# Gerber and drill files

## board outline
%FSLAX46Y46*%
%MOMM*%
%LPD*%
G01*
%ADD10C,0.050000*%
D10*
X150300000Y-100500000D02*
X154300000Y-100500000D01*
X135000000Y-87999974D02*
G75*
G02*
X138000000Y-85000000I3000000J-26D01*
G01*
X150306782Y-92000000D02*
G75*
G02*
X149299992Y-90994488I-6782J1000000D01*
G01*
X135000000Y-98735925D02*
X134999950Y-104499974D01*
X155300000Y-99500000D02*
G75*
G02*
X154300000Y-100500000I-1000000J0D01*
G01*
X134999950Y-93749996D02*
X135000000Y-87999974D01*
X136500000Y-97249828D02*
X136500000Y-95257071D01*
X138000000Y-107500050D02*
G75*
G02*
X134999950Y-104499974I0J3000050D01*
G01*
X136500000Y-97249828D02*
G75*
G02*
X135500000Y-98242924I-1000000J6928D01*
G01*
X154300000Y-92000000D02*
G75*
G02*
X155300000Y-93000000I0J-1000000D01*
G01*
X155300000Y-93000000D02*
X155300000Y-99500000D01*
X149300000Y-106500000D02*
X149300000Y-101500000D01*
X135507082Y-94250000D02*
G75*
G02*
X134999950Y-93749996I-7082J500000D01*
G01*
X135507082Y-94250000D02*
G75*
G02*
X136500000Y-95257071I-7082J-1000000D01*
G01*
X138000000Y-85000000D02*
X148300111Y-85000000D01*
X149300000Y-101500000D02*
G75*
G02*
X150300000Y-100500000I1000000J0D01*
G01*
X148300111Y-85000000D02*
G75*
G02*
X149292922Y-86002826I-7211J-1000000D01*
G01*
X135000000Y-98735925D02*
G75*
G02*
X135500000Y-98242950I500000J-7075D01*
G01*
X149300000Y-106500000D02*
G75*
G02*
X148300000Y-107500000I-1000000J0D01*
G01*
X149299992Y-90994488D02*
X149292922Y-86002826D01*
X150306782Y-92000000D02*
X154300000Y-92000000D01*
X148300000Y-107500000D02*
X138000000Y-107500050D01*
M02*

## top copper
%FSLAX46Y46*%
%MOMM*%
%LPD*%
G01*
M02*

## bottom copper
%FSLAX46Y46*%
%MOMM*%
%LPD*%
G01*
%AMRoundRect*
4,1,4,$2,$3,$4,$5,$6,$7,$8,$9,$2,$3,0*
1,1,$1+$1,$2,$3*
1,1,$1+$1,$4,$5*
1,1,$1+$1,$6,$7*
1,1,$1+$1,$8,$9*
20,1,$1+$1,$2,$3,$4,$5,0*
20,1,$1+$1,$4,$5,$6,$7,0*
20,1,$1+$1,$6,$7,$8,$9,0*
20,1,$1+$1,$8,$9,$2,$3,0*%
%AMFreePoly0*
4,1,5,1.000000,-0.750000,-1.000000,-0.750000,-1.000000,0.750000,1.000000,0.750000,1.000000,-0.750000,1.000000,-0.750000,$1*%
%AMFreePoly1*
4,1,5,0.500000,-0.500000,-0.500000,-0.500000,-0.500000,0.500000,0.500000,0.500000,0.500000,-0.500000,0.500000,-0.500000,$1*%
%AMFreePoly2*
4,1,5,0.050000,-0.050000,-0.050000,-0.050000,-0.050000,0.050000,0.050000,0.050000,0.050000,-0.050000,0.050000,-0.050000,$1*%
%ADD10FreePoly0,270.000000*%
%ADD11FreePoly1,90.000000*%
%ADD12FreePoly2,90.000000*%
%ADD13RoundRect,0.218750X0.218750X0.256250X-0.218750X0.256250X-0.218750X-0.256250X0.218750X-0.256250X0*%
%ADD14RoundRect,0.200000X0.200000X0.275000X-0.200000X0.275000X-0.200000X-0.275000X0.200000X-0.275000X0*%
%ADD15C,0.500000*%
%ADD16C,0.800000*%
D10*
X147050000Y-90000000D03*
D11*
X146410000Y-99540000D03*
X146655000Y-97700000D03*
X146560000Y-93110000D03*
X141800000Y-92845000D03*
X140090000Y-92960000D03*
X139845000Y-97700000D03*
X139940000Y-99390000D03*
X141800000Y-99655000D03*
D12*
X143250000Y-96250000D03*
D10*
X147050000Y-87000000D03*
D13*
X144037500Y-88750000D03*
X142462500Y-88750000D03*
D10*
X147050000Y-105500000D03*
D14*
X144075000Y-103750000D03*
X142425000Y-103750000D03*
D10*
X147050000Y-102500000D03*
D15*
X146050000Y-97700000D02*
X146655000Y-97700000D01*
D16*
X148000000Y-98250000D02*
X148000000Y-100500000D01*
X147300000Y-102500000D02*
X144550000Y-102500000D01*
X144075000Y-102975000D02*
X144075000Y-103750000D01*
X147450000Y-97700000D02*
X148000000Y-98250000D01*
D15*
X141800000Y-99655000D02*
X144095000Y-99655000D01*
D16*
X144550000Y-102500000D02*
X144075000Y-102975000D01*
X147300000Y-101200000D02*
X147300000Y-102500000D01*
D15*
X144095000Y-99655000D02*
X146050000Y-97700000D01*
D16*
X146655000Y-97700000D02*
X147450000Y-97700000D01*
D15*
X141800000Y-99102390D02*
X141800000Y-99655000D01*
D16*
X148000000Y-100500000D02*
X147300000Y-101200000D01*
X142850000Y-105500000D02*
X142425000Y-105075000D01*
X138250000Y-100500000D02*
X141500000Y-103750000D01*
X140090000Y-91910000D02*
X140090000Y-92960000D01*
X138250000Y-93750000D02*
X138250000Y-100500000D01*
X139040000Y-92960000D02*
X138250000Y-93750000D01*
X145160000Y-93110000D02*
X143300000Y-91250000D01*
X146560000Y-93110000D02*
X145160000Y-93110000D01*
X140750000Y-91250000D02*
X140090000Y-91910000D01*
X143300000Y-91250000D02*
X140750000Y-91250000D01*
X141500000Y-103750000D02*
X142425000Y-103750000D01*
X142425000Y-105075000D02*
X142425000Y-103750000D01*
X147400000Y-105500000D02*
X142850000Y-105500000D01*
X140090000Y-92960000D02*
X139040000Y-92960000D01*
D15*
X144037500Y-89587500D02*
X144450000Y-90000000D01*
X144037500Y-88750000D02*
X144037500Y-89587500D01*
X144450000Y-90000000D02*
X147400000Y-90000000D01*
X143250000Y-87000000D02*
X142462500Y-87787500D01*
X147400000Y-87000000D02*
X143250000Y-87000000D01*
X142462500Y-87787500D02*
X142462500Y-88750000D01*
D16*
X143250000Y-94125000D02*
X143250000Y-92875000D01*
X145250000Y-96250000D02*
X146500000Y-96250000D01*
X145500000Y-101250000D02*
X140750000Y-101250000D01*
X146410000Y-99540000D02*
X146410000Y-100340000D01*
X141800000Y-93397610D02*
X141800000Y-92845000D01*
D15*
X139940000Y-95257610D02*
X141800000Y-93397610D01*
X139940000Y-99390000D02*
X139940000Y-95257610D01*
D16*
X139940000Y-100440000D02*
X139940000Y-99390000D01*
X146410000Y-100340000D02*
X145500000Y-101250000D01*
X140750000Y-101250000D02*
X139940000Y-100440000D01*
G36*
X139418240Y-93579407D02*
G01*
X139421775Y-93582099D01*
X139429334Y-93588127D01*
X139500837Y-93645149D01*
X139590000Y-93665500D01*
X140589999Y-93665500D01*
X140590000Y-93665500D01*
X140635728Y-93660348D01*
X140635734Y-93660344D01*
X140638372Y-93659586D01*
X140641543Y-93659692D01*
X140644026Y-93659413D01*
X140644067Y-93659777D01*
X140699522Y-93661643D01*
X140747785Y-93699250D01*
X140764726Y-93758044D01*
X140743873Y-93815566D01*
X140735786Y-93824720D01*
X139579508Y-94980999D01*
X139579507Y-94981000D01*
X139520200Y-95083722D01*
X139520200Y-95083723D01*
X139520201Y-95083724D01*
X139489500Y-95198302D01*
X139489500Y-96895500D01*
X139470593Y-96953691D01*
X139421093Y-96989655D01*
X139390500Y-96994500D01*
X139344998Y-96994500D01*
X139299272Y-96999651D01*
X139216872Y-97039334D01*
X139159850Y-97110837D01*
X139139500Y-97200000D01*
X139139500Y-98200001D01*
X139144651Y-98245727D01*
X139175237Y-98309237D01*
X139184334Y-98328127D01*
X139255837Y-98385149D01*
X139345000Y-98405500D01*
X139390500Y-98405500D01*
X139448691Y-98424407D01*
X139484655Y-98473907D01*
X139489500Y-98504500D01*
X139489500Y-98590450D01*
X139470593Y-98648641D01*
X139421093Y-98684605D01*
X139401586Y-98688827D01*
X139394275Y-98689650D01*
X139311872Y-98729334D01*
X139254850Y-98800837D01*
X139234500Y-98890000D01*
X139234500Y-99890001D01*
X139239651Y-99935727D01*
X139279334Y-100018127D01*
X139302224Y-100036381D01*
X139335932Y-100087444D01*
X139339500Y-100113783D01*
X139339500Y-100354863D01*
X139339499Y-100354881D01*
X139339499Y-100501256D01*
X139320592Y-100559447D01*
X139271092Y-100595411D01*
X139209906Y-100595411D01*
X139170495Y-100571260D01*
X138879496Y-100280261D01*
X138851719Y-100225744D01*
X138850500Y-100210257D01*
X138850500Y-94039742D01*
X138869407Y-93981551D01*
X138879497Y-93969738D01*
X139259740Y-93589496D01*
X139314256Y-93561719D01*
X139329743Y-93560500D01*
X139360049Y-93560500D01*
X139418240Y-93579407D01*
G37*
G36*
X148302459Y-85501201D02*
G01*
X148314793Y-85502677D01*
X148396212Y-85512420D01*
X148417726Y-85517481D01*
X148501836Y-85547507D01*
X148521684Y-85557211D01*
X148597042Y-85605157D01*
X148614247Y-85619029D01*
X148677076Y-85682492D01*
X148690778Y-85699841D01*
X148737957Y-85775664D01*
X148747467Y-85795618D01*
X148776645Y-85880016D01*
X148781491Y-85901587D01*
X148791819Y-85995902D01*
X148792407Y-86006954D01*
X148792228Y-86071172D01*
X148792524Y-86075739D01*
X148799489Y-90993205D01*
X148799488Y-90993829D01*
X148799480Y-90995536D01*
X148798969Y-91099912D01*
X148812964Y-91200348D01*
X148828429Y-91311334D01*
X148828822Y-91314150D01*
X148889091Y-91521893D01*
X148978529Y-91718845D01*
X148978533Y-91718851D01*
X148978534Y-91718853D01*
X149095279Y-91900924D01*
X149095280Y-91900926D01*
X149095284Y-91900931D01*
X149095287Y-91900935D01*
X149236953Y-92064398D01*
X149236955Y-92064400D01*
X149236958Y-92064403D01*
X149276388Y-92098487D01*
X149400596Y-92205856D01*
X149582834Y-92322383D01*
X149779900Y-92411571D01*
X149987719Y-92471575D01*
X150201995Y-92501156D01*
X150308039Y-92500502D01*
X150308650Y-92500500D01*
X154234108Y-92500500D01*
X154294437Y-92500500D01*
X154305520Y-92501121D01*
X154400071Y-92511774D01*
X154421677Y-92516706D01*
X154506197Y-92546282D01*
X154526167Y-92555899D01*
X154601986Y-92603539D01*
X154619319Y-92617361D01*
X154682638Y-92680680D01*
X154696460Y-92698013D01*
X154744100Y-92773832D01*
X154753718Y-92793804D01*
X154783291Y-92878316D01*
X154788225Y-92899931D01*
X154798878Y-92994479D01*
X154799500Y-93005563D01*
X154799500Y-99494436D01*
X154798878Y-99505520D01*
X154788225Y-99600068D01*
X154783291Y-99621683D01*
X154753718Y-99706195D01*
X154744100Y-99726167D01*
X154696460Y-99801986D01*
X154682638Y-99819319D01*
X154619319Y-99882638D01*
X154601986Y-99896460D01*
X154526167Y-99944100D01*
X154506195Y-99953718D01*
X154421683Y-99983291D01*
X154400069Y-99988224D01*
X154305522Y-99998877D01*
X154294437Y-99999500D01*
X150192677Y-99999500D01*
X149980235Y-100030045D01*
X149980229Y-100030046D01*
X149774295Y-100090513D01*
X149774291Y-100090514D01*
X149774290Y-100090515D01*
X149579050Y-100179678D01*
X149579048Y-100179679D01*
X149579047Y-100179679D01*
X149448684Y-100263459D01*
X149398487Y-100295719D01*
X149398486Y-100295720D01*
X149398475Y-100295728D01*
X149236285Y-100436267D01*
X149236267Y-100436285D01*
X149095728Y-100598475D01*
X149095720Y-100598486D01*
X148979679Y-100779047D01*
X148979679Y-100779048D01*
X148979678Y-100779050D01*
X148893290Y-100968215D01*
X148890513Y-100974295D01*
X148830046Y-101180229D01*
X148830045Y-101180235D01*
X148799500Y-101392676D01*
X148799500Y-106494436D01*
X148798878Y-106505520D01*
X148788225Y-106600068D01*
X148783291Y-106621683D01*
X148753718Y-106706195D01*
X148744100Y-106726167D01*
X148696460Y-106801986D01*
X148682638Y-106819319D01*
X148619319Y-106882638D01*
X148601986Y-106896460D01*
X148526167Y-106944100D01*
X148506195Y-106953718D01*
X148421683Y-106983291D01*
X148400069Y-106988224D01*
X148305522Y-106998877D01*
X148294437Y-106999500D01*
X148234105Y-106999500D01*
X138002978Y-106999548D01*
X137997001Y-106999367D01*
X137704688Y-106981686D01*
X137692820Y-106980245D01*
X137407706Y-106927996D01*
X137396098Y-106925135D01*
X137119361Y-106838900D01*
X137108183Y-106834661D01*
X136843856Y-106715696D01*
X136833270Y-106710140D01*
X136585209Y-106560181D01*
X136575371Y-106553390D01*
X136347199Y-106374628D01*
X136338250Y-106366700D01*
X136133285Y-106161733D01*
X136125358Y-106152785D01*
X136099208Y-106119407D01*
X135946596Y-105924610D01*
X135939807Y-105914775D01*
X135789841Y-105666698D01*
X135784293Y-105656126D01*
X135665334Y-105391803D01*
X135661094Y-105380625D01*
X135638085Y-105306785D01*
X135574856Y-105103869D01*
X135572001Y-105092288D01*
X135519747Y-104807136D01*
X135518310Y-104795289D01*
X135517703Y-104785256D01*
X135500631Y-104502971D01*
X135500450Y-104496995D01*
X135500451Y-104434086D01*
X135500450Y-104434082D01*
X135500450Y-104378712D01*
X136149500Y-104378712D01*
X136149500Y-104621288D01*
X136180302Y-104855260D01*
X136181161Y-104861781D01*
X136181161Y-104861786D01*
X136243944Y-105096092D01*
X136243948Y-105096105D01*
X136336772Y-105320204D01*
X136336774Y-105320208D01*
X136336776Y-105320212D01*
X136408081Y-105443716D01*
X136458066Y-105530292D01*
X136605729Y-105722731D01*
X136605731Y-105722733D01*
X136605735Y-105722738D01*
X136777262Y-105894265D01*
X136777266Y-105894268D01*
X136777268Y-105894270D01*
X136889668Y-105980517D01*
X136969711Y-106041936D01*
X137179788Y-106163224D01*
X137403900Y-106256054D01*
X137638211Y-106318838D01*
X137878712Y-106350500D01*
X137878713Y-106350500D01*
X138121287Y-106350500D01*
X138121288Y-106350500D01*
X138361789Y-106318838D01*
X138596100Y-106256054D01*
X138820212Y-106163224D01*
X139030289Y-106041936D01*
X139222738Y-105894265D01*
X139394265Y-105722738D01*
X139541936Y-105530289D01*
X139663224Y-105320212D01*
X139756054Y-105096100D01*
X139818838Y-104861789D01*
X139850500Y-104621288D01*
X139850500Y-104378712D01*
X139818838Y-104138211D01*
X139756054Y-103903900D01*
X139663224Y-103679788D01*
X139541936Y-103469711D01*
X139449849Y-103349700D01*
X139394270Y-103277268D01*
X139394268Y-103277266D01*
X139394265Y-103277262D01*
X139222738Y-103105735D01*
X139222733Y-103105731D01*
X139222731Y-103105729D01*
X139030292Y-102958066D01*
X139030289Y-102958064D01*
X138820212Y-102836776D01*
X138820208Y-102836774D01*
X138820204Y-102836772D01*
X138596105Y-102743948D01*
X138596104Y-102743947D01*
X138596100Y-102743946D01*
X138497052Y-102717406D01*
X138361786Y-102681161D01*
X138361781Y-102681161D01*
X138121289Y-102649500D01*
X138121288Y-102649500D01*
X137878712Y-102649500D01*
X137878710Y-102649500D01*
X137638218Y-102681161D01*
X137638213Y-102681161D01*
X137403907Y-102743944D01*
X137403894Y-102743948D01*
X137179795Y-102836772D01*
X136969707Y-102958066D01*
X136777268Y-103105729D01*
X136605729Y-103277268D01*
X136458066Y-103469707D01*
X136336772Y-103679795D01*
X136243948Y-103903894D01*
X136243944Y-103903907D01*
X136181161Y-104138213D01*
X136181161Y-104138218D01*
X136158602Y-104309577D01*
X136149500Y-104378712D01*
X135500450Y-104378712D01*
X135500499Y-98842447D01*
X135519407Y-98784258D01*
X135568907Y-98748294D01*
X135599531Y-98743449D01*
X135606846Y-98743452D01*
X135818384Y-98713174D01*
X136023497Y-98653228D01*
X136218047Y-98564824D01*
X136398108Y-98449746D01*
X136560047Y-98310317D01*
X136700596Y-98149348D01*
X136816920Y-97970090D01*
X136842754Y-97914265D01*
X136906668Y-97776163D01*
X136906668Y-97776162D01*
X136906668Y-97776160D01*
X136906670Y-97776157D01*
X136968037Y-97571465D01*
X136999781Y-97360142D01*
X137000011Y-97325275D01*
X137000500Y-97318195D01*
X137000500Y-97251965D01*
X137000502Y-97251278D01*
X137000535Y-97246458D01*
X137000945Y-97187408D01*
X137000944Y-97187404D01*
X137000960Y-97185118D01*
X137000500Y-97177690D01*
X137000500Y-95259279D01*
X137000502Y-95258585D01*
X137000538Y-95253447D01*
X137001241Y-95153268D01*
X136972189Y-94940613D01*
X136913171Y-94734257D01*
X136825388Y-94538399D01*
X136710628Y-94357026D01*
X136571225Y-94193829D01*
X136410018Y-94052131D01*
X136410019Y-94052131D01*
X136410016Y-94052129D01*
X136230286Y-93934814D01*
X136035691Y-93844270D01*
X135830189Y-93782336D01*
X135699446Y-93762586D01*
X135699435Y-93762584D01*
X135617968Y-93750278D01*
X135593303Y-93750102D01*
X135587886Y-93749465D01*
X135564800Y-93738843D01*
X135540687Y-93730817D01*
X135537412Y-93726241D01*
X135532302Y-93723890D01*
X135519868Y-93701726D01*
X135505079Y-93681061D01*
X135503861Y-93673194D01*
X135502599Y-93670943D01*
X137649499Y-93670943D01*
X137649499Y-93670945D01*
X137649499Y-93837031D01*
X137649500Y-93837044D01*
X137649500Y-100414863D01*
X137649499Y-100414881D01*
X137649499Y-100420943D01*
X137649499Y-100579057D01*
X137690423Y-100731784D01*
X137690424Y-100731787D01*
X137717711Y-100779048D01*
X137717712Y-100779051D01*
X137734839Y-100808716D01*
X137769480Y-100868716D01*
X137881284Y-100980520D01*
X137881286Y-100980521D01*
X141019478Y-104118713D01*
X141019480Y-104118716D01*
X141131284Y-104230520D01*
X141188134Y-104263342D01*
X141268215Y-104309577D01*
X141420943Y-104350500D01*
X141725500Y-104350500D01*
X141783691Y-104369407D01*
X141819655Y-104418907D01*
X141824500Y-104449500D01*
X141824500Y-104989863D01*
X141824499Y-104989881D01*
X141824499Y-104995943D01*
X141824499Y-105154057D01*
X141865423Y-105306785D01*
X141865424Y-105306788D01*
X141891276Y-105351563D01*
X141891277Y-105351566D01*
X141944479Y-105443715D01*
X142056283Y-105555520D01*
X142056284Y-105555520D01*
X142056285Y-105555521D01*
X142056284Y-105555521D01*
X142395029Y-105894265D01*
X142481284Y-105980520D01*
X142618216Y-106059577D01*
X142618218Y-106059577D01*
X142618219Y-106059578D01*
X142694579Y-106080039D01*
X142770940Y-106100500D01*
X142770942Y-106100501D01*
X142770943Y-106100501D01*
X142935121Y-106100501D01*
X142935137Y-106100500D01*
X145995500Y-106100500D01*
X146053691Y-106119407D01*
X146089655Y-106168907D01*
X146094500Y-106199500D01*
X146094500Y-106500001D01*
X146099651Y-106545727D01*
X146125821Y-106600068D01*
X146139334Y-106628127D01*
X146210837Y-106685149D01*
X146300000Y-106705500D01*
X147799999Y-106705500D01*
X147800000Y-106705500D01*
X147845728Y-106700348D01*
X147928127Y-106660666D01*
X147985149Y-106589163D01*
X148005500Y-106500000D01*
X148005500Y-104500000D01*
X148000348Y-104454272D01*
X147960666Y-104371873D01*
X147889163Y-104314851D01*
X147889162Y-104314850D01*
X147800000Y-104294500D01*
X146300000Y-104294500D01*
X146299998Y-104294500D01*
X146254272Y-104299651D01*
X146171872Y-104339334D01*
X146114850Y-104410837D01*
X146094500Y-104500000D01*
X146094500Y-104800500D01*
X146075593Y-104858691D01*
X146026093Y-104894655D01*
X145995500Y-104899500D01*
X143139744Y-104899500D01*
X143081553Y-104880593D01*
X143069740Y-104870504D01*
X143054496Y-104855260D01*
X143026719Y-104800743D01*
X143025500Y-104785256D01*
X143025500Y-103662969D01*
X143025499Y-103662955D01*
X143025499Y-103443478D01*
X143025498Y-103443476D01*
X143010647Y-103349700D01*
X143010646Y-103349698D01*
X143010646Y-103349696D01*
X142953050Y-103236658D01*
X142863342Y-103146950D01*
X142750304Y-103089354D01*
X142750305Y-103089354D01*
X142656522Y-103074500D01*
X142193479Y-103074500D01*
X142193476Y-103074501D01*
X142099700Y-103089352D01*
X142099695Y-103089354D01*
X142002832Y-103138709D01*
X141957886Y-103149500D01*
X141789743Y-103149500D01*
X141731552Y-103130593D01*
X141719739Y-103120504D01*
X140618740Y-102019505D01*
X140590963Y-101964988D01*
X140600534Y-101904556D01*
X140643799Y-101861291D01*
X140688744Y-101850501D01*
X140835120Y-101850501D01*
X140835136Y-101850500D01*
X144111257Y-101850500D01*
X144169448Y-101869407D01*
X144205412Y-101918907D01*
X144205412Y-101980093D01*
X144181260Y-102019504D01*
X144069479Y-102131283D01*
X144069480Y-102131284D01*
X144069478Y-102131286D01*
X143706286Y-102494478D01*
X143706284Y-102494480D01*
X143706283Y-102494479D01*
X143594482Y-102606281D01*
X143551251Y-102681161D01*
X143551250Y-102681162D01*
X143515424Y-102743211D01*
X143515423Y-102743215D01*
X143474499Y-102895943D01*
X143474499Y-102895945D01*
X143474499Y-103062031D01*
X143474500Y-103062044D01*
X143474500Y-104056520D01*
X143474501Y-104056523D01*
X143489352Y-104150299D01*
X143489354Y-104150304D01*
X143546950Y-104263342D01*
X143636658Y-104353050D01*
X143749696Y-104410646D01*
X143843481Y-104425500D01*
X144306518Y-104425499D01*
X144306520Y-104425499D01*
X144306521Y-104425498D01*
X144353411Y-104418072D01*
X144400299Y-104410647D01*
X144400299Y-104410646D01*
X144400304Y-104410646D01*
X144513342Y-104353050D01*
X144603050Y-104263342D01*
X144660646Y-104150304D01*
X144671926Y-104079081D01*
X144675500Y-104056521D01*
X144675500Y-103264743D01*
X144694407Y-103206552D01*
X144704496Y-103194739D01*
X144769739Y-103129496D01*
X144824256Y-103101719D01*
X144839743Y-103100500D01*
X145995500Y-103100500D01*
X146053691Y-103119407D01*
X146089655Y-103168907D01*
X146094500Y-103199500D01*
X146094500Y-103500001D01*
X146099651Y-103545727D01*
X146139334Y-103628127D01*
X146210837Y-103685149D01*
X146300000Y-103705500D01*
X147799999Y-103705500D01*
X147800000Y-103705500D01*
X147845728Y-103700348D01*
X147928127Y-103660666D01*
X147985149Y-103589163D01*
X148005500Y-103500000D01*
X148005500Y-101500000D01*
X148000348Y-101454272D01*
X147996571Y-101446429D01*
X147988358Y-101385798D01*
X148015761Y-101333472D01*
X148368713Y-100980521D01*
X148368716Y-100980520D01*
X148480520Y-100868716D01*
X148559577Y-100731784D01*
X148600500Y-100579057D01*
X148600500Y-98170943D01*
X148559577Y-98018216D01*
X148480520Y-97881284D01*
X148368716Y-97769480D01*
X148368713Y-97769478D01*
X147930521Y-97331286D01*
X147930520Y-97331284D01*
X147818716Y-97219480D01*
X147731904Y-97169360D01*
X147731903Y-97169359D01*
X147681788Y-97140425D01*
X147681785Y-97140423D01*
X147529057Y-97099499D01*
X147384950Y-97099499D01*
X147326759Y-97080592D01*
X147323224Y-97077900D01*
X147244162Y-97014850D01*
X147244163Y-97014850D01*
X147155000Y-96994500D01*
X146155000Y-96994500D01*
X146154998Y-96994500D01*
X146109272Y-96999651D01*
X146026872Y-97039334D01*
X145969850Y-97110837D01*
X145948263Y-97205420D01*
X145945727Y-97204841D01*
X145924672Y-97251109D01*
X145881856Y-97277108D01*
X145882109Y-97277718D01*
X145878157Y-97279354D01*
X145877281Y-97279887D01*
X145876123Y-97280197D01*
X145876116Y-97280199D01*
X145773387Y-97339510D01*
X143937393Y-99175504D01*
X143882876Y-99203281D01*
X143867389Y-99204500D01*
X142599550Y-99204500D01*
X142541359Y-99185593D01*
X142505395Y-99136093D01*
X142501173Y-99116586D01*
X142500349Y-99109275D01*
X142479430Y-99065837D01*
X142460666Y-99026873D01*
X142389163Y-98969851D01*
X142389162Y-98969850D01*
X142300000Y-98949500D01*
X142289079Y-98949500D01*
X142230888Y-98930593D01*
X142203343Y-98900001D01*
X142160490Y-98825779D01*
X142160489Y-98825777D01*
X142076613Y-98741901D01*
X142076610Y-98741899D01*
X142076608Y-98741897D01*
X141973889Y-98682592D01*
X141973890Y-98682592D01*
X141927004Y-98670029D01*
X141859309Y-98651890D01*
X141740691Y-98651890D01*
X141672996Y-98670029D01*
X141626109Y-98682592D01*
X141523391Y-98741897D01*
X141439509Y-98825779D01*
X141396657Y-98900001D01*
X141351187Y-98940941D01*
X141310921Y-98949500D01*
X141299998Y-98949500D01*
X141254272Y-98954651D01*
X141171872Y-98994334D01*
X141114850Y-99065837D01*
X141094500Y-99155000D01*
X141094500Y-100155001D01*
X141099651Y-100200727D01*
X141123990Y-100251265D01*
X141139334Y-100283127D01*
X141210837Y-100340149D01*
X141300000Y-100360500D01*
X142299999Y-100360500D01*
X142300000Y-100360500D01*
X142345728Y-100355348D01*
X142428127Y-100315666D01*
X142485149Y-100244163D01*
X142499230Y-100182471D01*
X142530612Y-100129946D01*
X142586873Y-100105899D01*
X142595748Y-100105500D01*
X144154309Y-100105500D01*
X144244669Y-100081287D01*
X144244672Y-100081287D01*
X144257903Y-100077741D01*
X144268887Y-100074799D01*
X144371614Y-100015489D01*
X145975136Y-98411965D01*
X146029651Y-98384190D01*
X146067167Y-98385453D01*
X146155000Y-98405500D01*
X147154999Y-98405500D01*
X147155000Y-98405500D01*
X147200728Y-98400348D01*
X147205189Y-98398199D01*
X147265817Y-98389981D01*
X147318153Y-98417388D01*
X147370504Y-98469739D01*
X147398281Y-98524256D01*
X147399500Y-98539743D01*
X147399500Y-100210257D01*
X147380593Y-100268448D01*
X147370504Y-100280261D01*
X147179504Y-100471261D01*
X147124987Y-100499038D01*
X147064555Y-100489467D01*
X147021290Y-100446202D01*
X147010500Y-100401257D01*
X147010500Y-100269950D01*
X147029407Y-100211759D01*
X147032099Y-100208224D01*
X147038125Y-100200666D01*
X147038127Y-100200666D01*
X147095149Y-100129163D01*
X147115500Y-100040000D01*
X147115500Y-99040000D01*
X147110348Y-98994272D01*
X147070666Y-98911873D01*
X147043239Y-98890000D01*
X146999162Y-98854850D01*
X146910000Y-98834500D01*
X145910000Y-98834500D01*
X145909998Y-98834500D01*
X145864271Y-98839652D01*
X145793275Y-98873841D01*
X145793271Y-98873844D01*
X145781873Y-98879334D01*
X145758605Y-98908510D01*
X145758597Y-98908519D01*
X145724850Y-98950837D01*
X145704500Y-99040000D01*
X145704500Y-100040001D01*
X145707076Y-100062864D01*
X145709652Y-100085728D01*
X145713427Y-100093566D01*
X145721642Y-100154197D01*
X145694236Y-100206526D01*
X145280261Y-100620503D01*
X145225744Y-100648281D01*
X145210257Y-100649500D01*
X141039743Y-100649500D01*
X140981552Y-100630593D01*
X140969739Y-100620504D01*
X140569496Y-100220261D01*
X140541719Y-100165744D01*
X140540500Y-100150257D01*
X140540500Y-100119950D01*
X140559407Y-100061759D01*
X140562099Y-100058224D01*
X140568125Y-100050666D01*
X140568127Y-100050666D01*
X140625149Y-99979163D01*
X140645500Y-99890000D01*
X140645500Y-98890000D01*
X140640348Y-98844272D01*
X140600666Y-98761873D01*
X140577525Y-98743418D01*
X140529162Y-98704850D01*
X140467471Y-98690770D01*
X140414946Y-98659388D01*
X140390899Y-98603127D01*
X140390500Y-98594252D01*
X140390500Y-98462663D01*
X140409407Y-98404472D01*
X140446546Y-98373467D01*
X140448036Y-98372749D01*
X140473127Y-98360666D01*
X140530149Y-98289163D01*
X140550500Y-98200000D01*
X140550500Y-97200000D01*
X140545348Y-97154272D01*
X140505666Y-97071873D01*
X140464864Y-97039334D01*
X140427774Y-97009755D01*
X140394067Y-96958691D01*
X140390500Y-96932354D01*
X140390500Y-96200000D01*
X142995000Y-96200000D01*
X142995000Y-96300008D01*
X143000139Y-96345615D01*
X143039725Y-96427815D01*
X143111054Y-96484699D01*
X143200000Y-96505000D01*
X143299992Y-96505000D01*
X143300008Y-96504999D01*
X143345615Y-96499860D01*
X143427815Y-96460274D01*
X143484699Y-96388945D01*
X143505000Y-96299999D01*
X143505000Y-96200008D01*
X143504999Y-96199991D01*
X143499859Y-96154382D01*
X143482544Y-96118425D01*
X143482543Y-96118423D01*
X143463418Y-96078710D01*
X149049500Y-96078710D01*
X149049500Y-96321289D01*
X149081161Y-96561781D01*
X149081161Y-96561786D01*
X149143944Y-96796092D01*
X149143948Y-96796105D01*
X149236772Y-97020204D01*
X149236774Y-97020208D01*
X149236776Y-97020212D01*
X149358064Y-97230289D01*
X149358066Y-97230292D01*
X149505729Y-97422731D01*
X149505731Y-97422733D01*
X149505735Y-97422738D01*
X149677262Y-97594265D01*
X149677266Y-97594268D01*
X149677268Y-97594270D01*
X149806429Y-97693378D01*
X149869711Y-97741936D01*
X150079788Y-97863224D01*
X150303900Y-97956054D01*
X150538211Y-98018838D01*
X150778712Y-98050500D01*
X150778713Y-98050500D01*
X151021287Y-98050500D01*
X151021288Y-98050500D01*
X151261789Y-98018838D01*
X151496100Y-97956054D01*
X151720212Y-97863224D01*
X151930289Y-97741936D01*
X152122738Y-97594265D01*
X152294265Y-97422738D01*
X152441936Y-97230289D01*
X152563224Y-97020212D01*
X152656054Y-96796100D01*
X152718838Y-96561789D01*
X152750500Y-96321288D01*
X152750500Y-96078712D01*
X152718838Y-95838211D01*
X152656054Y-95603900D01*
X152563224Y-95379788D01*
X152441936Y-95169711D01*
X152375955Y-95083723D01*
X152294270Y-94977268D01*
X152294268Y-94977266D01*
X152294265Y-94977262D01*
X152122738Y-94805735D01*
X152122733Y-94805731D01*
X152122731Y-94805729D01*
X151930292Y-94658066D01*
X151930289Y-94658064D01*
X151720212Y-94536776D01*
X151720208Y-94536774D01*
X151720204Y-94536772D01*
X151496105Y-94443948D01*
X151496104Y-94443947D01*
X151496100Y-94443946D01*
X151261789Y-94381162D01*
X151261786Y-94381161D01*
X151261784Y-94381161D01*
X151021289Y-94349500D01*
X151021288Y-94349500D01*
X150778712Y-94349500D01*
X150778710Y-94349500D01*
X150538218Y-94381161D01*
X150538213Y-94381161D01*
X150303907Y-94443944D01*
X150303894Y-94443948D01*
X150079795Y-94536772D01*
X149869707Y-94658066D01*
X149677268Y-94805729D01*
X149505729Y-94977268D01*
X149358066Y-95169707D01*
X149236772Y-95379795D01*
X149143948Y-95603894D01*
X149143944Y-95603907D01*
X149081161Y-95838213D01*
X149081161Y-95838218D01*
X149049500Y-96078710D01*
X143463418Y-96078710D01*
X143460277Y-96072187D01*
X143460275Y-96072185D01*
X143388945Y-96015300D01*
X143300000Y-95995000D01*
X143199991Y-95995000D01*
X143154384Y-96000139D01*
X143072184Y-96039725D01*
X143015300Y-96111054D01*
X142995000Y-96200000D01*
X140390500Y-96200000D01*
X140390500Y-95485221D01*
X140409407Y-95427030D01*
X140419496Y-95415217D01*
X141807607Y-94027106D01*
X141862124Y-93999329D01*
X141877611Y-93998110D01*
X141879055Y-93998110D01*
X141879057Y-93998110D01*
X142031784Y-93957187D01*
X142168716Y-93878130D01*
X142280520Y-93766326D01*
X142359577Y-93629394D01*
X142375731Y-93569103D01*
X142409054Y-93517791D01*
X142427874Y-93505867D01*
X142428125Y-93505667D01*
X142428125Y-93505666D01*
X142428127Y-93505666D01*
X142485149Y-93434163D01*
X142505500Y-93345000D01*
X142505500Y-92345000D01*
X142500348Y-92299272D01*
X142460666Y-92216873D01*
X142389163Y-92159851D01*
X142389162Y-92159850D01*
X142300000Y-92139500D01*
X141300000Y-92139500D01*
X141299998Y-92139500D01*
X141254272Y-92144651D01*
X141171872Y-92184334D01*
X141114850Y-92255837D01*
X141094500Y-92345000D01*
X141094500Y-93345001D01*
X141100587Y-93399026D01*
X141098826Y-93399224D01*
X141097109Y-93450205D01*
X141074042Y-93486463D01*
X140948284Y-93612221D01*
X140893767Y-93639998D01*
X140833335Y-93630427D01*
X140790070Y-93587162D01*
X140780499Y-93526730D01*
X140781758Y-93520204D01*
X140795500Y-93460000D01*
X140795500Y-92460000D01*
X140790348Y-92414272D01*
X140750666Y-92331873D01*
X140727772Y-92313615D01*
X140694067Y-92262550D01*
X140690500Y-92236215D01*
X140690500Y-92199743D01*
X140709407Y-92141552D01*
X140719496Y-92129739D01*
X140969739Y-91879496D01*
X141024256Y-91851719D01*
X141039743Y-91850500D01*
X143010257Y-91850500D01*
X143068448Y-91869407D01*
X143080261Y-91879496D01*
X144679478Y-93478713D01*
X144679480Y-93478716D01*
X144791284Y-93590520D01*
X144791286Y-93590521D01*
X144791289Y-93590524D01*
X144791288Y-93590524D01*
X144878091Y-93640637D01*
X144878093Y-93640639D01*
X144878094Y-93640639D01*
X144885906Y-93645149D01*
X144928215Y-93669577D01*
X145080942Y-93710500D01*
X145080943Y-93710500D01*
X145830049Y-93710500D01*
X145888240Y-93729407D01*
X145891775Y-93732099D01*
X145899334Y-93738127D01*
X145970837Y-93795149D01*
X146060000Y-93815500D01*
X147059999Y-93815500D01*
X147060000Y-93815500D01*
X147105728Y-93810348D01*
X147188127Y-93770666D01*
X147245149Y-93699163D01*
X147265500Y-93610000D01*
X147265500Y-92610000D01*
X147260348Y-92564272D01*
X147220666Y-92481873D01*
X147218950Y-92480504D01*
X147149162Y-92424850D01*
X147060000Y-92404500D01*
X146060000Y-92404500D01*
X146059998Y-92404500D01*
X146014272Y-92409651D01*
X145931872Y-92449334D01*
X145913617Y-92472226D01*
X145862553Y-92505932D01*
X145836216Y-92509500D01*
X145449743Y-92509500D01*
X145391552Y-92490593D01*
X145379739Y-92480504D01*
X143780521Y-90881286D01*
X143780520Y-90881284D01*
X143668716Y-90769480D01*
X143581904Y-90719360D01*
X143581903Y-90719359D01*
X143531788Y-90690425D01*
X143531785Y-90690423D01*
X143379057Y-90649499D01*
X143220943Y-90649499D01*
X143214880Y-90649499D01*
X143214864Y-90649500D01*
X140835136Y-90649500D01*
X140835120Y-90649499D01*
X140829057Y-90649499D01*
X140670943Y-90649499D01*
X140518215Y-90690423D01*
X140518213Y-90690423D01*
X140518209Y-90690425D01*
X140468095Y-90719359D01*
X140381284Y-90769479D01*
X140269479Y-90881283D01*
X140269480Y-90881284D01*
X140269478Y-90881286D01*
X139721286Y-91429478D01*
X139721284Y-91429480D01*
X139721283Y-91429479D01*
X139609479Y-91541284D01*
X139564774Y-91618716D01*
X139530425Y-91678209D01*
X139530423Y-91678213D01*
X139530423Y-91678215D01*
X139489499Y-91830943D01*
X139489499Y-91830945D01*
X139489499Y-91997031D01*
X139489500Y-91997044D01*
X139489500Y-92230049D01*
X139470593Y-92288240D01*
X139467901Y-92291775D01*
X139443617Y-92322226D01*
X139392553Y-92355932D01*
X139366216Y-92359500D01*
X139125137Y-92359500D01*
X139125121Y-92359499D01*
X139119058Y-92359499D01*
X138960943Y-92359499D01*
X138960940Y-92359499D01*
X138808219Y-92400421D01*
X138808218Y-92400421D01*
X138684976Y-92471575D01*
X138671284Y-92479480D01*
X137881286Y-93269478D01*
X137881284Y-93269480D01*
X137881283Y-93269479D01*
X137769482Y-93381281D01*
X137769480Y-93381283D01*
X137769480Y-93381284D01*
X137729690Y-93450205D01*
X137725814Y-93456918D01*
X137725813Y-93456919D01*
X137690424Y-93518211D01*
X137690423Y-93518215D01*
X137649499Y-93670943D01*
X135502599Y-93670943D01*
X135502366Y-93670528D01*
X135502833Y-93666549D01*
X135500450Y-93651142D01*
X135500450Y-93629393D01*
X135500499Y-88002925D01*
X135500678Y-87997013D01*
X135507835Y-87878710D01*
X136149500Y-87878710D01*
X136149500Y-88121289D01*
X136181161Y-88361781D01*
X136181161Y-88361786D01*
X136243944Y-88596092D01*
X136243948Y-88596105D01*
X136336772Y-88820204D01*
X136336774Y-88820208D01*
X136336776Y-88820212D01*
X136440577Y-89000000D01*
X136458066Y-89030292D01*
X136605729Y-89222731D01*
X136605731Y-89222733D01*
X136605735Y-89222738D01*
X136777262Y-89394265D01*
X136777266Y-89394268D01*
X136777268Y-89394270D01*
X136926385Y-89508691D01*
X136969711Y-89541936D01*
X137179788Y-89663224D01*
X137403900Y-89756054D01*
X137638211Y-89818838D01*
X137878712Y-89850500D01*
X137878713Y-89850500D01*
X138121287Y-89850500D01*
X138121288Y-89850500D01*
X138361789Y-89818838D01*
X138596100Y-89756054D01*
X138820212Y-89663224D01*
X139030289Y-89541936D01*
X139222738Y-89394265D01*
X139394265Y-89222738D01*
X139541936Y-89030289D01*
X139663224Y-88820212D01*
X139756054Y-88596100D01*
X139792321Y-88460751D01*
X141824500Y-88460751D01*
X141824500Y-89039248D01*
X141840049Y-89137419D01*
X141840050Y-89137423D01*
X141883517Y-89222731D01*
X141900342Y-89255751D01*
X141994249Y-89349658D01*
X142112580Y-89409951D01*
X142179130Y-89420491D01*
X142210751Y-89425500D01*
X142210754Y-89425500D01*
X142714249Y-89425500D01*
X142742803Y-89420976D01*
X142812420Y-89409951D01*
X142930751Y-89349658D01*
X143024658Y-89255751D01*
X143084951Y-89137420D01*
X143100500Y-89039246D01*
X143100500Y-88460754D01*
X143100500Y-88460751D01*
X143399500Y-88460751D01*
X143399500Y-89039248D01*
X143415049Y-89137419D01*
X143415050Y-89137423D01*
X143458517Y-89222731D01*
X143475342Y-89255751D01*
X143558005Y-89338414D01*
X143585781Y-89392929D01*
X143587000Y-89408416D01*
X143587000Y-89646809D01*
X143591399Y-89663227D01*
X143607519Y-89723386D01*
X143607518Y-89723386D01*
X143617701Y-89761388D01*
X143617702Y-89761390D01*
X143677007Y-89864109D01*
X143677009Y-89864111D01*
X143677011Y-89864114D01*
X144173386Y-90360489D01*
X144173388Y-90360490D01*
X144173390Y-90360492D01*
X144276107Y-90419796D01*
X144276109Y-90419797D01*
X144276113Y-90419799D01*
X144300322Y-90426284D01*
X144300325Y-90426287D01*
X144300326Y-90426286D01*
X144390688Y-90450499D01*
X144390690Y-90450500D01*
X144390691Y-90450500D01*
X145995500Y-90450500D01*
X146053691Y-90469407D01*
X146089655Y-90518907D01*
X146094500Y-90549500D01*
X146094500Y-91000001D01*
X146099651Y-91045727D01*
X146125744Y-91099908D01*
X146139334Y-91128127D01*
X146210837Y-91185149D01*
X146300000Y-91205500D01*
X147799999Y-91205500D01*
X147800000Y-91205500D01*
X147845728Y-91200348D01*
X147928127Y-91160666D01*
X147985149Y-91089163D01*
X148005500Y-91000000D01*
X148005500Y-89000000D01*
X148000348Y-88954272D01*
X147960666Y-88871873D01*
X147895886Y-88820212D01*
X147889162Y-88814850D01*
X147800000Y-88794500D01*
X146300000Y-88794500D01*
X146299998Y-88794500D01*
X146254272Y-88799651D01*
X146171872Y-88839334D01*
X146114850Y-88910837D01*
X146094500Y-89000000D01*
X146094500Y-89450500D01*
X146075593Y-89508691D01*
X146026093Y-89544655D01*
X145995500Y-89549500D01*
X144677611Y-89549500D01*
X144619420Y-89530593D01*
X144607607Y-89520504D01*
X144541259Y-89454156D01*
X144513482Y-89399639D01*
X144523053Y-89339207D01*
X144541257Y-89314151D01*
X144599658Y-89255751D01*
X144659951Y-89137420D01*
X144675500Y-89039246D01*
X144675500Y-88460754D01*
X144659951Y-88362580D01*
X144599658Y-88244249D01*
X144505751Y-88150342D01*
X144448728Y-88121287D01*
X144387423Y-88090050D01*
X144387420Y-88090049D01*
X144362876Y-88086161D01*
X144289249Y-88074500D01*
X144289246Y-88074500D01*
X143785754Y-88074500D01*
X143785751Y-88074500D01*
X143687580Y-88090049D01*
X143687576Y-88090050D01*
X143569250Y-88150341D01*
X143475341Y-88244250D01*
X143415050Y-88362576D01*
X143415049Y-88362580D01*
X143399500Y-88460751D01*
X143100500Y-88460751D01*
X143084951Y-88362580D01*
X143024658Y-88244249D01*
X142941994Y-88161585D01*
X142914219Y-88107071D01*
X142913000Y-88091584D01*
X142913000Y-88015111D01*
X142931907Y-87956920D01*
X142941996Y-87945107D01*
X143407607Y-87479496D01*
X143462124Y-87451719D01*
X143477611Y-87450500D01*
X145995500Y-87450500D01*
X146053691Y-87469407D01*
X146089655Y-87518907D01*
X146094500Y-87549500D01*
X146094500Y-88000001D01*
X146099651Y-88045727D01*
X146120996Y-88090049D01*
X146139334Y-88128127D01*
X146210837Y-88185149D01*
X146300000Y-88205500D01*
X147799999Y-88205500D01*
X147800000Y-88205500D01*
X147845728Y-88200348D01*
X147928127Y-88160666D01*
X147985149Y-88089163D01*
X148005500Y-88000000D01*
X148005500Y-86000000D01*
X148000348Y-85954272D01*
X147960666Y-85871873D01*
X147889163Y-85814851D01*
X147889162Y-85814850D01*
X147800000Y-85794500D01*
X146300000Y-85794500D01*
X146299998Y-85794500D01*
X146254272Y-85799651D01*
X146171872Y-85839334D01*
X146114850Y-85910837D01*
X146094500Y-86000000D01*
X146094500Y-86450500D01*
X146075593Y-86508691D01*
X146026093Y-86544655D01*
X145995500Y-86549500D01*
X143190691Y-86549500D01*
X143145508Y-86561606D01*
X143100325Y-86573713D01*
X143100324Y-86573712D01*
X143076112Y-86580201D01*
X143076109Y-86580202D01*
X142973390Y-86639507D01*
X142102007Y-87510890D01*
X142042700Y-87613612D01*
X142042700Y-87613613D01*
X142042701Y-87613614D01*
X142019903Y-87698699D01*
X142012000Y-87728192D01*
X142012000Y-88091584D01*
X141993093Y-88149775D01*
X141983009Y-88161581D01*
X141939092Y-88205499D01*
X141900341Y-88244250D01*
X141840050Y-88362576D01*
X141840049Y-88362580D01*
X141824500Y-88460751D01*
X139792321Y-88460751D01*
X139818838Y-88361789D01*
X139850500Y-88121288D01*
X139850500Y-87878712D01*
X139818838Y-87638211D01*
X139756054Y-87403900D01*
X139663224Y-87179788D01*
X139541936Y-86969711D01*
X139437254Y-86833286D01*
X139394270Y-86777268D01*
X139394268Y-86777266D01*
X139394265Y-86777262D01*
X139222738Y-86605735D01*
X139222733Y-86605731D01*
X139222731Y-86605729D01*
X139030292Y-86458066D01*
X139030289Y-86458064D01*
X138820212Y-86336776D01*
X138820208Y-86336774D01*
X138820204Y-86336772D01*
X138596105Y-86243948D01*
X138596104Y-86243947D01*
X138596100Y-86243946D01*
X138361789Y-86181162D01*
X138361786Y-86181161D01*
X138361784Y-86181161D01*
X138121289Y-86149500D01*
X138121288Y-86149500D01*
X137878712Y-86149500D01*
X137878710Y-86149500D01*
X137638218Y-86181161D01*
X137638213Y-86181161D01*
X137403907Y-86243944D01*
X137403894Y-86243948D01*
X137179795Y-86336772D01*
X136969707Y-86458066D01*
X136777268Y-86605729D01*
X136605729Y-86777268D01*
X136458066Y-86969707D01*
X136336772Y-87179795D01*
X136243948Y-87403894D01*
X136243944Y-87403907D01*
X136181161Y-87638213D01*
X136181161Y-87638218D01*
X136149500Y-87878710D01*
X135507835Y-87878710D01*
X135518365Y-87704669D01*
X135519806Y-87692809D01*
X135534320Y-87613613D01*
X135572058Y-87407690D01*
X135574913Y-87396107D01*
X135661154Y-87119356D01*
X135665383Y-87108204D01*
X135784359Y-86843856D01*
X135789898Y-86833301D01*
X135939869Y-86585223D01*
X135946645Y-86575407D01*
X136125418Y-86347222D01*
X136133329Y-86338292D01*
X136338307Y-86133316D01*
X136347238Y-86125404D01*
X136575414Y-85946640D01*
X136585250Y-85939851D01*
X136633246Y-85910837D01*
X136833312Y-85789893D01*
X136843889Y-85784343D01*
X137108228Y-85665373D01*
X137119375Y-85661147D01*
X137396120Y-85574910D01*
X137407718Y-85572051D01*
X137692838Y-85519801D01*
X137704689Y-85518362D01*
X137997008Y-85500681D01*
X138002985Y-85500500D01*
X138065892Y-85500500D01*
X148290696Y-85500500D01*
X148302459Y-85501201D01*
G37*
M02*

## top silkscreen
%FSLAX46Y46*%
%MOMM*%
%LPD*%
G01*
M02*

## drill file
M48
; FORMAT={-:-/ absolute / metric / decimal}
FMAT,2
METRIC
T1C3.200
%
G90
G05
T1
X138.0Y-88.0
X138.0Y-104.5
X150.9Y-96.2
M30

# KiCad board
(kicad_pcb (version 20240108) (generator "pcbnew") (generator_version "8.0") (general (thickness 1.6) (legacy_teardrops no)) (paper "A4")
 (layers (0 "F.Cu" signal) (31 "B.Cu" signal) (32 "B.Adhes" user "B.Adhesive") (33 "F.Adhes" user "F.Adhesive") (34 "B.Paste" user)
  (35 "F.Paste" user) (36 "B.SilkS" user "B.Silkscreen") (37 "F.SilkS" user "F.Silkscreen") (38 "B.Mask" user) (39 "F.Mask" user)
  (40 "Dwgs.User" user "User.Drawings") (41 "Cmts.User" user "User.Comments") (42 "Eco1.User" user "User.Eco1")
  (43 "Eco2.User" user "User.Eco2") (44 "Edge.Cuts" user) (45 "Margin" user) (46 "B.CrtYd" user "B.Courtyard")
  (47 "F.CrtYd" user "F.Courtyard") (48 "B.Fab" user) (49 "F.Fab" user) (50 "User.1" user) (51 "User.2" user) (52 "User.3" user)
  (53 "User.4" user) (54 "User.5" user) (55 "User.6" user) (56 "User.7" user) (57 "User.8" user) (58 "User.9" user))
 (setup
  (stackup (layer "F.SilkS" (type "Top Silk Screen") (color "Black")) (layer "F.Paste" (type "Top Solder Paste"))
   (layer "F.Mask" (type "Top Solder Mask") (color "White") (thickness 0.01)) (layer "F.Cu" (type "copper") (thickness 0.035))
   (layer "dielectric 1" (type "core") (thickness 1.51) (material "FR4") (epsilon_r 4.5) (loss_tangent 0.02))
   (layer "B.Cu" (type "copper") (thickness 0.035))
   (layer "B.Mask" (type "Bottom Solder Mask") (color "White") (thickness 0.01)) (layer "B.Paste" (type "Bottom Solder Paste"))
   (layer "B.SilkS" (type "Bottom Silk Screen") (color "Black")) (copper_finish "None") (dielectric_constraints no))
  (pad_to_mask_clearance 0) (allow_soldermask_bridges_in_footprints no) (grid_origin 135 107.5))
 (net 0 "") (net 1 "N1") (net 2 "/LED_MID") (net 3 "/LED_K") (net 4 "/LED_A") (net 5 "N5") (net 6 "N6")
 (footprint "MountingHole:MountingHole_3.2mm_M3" (layer "F.Cu") (at 138 104.5)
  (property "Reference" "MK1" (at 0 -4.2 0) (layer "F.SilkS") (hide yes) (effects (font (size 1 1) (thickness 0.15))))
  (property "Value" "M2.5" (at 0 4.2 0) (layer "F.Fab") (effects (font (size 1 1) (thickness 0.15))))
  (pad "" np_thru_hole circle (at 0 0) (size 3.2 3.2) (drill 3.2) (layers "*.Cu" "*.Mask")))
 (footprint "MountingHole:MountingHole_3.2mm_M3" (layer "F.Cu") (at 150.9 96.2)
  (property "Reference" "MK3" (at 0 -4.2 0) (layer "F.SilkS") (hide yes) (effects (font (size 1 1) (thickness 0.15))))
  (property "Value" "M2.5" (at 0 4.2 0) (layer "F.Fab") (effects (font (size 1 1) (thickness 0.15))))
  (pad "" np_thru_hole circle (at 0 0) (size 3.2 3.2) (drill 3.2) (layers "*.Cu" "*.Mask")))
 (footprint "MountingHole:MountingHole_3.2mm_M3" (layer "F.Cu") (at 138 88)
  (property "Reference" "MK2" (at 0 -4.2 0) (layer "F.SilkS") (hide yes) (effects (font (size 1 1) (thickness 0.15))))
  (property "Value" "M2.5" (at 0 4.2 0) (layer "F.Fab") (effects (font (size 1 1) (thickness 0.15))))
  (pad "" np_thru_hole circle (at 0 0) (size 3.2 3.2) (drill 3.2) (layers "*.Cu" "*.Mask")))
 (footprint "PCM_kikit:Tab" (layer "F.Cu") (at 143.5 85 -90)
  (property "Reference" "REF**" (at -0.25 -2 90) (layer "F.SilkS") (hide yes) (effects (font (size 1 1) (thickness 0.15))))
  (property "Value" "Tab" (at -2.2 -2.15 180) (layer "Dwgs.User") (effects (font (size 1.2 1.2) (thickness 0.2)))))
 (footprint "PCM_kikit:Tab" (layer "F.Cu") (at 143.5 107.5 90)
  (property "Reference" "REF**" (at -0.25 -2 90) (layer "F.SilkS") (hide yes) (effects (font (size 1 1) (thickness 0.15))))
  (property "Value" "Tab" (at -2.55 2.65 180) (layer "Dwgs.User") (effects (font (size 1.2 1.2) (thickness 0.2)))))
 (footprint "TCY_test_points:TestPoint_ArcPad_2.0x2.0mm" (layer "B.Cu") (at 147.05 90 -90)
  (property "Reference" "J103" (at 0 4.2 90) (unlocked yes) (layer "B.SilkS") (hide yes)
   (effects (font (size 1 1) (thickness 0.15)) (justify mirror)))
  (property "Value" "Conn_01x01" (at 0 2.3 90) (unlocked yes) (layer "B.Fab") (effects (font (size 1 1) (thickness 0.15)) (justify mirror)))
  (pad "1" smd custom (at 0 0 270) (size 2 1.5) (layers "B.Cu" "B.Paste" "B.Mask") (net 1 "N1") (options (clearance outline) (anchor rect))
   (primitives)))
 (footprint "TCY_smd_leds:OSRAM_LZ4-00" (layer "B.Cu") (at 143.25 96.25 90)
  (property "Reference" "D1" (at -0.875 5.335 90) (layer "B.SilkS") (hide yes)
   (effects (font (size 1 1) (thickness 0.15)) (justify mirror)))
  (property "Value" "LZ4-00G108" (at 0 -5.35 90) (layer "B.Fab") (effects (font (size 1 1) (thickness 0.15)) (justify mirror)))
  (pad "1" smd custom (at -3.29 3.16 90) (size 1 1) (layers "B.Cu") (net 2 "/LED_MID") (options (clearance outline) (anchor rect))
   (primitives))
  (pad "2" smd custom (at -1.45 3.405 90) (size 1 1) (layers "B.Cu") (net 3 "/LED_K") (zone_connect 2)
   (options (clearance outline) (anchor rect)) (primitives))
  (pad "3" smd custom (at 3.14 3.31 90) (size 1 1) (layers "B.Cu") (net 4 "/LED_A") (options (clearance outline) (anchor rect)) (primitives))
  (pad "4" smd custom (at 3.405 -1.45 90) (size 1 1) (layers "B.Cu") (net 2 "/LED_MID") (zone_connect 2)
   (options (clearance outline) (anchor rect)) (primitives))
  (pad "5" smd custom (at 3.29 -3.16 90) (size 1 1) (layers "B.Cu") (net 4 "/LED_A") (options (clearance outline) (anchor rect))
   (primitives))
  (pad "6" smd custom (at -1.45 -3.405 90) (size 1 1) (layers "B.Cu") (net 2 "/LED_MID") (zone_connect 2)
   (options (clearance outline) (anchor rect)) (primitives))
  (pad "7" smd custom (at -3.14 -3.31 90) (size 1 1) (layers "B.Cu") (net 2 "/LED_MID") (options (clearance outline) (anchor rect))
   (primitives))
  (pad "8" smd custom (at -3.405 -1.45 90) (size 1 1) (layers "B.Cu") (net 3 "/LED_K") (zone_connect 2)
   (options (clearance outline) (anchor rect)) (primitives))
  (pad "9" smd custom (at 0 0 90) (size 0.1 0.1) (layers "B.Cu") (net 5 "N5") (options (clearance outline) (anchor rect)) (primitives)))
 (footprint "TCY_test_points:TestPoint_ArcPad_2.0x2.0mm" (layer "B.Cu") (at 147.05 87 -90)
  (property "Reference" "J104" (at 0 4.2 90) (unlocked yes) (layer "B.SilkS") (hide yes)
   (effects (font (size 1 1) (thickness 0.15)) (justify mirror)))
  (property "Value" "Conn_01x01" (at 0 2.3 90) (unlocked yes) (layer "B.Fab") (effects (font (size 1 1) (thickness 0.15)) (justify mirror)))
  (pad "1" smd custom (at 0 0 270) (size 2 1.5) (layers "B.Cu" "B.Paste" "B.Mask") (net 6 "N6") (options (clearance outline) (anchor rect))
   (primitives)))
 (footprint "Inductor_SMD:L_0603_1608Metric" (layer "B.Cu") (at 143.25 88.75 180)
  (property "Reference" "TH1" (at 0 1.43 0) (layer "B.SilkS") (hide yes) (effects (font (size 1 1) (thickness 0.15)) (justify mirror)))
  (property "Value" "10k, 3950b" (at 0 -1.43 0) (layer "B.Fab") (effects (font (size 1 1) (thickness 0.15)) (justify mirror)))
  (pad "1" smd roundrect (at -0.7875 0 180) (size 0.875 0.95) (layers "B.Cu" "B.Paste" "B.Mask") (roundrect_rratio 0.25) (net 1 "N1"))
  (pad "2" smd roundrect (at 0.7875 0 180) (size 0.875 0.95) (layers "B.Cu" "B.Paste" "B.Mask") (roundrect_rratio 0.25) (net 6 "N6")))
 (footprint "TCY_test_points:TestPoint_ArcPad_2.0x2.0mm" (layer "B.Cu") (at 147.05 105.5 -90)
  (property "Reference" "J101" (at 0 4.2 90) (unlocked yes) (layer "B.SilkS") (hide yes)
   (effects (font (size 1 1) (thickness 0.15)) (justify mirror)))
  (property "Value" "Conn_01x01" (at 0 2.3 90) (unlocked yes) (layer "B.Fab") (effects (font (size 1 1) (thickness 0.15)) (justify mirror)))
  (pad "1" smd custom (at 0 0 270) (size 2 1.5) (layers "B.Cu" "B.Paste" "B.Mask") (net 4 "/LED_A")
   (options (clearance outline) (anchor rect)) (primitives)))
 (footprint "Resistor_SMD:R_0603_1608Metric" (layer "B.Cu") (at 143.25 103.75 180)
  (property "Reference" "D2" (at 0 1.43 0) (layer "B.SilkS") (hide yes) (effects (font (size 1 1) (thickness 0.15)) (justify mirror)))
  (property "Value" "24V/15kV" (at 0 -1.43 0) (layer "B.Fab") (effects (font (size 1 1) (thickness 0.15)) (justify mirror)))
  (pad "1" smd roundrect (at -0.825 0 180) (size 0.8 0.95) (layers "B.Cu" "B.Paste" "B.Mask") (roundrect_rratio 0.25) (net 3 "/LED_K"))
  (pad "2" smd roundrect (at 0.825 0 180) (size 0.8 0.95) (layers "B.Cu" "B.Paste" "B.Mask") (roundrect_rratio 0.25) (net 4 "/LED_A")))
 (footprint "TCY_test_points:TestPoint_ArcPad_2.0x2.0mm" (layer "B.Cu") (at 147.05 102.5 -90)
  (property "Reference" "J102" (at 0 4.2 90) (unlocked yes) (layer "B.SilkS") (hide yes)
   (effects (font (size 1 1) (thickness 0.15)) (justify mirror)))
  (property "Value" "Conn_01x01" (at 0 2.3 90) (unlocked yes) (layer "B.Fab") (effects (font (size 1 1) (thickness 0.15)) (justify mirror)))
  (pad "1" smd custom (at 0 0 270) (size 2 1.5) (layers "B.Cu" "B.Paste" "B.Mask") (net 3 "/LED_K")
   (options (clearance outline) (anchor rect)) (primitives)))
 (gr_line (start 150.3 100.5) (end 154.3 100.5) (stroke (width 0.05) (type default)) (layer "Edge.Cuts"))
 (gr_arc (start 135 87.999974) (mid 135.87868 85.87868) (end 138 85) (stroke (width 0.05) (type default)) (layer "Edge.Cuts"))
 (gr_arc (start 150.306782 92) (mid 149.590392 91.704607) (end 149.299992 90.994488) (stroke (width 0.05) (type default))
  (layer "Edge.Cuts"))
 (gr_line (start 135 98.735925) (end 134.99995 104.499974) (stroke (width 0.05) (type default)) (layer "Edge.Cuts"))
 (gr_arc (start 155.3 99.5) (mid 155.007107 100.207107) (end 154.3 100.5) (stroke (width 0.05) (type default)) (layer "Edge.Cuts"))
 (gr_line (start 134.99995 93.749996) (end 135 87.999974) (stroke (width 0.05) (type default)) (layer "Edge.Cuts"))
 (gr_line (start 136.5 97.249828) (end 136.5 95.257071) (stroke (width 0.05) (type default)) (layer "Edge.Cuts"))
 (gr_arc (start 138 107.50005) (mid 135.878635 106.621347) (end 134.99995 104.499974) (stroke (width 0.05) (type default))
  (layer "Edge.Cuts"))
 (gr_arc (start 136.5 97.249828) (mid 136.204607 97.952526) (end 135.5 98.242918) (stroke (width 0.05) (type default)) (layer "Edge.Cuts"))
 (gr_arc (start 154.3 92) (mid 155.007107 92.292893) (end 155.3 93) (stroke (width 0.05) (type default)) (layer "Edge.Cuts"))
 (gr_line (start 155.3 93) (end 155.3 99.5) (stroke (width 0.05) (type default)) (layer "Edge.Cuts"))
 (gr_line (start 149.3 106.5) (end 149.3 101.5) (stroke (width 0.05) (type default)) (layer "Edge.Cuts"))
 (gr_arc (start 135.507082 94.25) (mid 135.148924 94.106084) (end 134.99995 93.749996) (stroke (width 0.05) (type default))
  (layer "Edge.Cuts"))
 (gr_arc (start 135.507082 94.25) (mid 136.209608 94.545393) (end 136.5 95.257071) (stroke (width 0.05) (type default)) (layer "Edge.Cuts"))
 (gr_line (start 138 85) (end 148.300111 85) (stroke (width 0.05) (type default)) (layer "Edge.Cuts"))
 (gr_arc (start 149.3 101.5) (mid 149.592893 100.792893) (end 150.3 100.5) (stroke (width 0.05) (type default)) (layer "Edge.Cuts"))
 (gr_arc (start 148.300111 85) (mid 149.002526 85.295393) (end 149.292922 86.002826) (stroke (width 0.05) (type default))
  (layer "Edge.Cuts"))
 (gr_arc (start 135 98.735925) (mid 135.143916 98.391892) (end 135.5 98.242918) (stroke (width 0.05) (type default)) (layer "Edge.Cuts"))
 (gr_arc (start 149.3 106.5) (mid 149.007107 107.207107) (end 148.3 107.5) (stroke (width 0.05) (type default)) (layer "Edge.Cuts"))
 (gr_line (start 149.299992 90.994488) (end 149.292922 86.002826) (stroke (width 0.05) (type default)) (layer "Edge.Cuts"))
 (gr_line (start 150.306782 92) (end 154.3 92) (stroke (width 0.05) (type default)) (layer "Edge.Cuts"))
 (gr_line (start 148.3 107.5) (end 138 107.50005) (stroke (width 0.05) (type default)) (layer "Edge.Cuts"))
 (segment (start 146.05 97.7) (end 146.655 97.7) (width 0.5) (layer "B.Cu") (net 3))
 (segment (start 148 98.25) (end 148 100.5) (width 0.8) (layer "B.Cu") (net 3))
 (segment (start 147.3 102.5) (end 144.55 102.5) (width 0.8) (layer "B.Cu") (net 3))
 (segment (start 144.075 102.975) (end 144.075 103.75) (width 0.8) (layer "B.Cu") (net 3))
 (segment (start 147.45 97.7) (end 148 98.25) (width 0.8) (layer "B.Cu") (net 3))
 (segment (start 141.8 99.655) (end 144.095 99.655) (width 0.5) (layer "B.Cu") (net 3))
 (segment (start 144.55 102.5) (end 144.075 102.975) (width 0.8) (layer "B.Cu") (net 3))
 (segment (start 147.3 101.2) (end 147.3 102.5) (width 0.8) (layer "B.Cu") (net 3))
 (segment (start 144.095 99.655) (end 146.05 97.7) (width 0.5) (layer "B.Cu") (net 3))
 (segment (start 146.655 97.7) (end 147.45 97.7) (width 0.8) (layer "B.Cu") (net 3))
 (segment (start 141.8 99.10239) (end 141.8 99.655) (width 0.5) (layer "B.Cu") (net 3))
 (segment (start 148 100.5) (end 147.3 101.2) (width 0.8) (layer "B.Cu") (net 3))
 (segment (start 142.85 105.5) (end 142.425 105.075) (width 0.8) (layer "B.Cu") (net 4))
 (segment (start 138.25 100.5) (end 141.5 103.75) (width 0.8) (layer "B.Cu") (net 4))
 (segment (start 140.09 91.91) (end 140.09 92.96) (width 0.8) (layer "B.Cu") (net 4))
 (segment (start 138.25 93.75) (end 138.25 100.5) (width 0.8) (layer "B.Cu") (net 4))
 (segment (start 139.04 92.96) (end 138.25 93.75) (width 0.8) (layer "B.Cu") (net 4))
 (segment (start 145.16 93.11) (end 143.3 91.25) (width 0.8) (layer "B.Cu") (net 4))
 (segment (start 146.56 93.11) (end 145.16 93.11) (width 0.8) (layer "B.Cu") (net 4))
 (segment (start 140.75 91.25) (end 140.09 91.91) (width 0.8) (layer "B.Cu") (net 4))
 (segment (start 143.3 91.25) (end 140.75 91.25) (width 0.8) (layer "B.Cu") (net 4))
 (segment (start 141.5 103.75) (end 142.425 103.75) (width 0.8) (layer "B.Cu") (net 4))
 (segment (start 142.425 105.075) (end 142.425 103.75) (width 0.8) (layer "B.Cu") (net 4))
 (segment (start 147.4 105.5) (end 142.85 105.5) (width 0.8) (layer "B.Cu") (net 4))
 (segment (start 140.09 92.96) (end 139.04 92.96) (width 0.8) (layer "B.Cu") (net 4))
 (segment (start 144.0375 89.5875) (end 144.45 90) (width 0.5) (layer "B.Cu") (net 1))
 (segment (start 144.0375 88.75) (end 144.0375 89.5875) (width 0.5) (layer "B.Cu") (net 1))
 (segment (start 144.45 90) (end 147.4 90) (width 0.5) (layer "B.Cu") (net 1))
 (segment (start 143.25 87) (end 142.4625 87.7875) (width 0.5) (layer "B.Cu") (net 6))
 (segment (start 147.4 87) (end 143.25 87) (width 0.5) (layer "B.Cu") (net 6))
 (segment (start 142.4625 87.7875) (end 142.4625 88.75) (width 0.5) (layer "B.Cu") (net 6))
 (segment (start 143.25 94.125) (end 143.25 92.875) (width 0.8) (layer "B.Cu") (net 5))
 (segment (start 145.25 96.25) (end 146.5 96.25) (width 0.8) (layer "B.Cu") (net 5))
 (segment (start 145.5 101.25) (end 140.75 101.25) (width 0.8) (layer "B.Cu") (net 2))
 (segment (start 146.41 99.54) (end 146.41 100.34) (width 0.8) (layer "B.Cu") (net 2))
 (segment (start 141.8 93.39761) (end 141.8 92.845) (width 0.8) (layer "B.Cu") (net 2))
 (segment (start 139.94 95.25761) (end 141.8 93.39761) (width 0.5) (layer "B.Cu") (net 2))
 (segment (start 139.94 99.39) (end 139.94 95.25761) (width 0.5) (layer "B.Cu") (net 2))
 (segment (start 139.94 100.44) (end 139.94 99.39) (width 0.8) (layer "B.Cu") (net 2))
 (segment (start 146.41 100.34) (end 145.5 101.25) (width 0.8) (layer "B.Cu") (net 2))
 (segment (start 140.75 101.25) (end 139.94 100.44) (width 0.8) (layer "B.Cu") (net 2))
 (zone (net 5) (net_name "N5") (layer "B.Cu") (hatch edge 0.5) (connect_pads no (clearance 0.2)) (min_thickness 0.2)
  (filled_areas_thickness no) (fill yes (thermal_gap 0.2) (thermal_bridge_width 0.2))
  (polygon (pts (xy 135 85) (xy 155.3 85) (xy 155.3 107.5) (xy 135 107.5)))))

